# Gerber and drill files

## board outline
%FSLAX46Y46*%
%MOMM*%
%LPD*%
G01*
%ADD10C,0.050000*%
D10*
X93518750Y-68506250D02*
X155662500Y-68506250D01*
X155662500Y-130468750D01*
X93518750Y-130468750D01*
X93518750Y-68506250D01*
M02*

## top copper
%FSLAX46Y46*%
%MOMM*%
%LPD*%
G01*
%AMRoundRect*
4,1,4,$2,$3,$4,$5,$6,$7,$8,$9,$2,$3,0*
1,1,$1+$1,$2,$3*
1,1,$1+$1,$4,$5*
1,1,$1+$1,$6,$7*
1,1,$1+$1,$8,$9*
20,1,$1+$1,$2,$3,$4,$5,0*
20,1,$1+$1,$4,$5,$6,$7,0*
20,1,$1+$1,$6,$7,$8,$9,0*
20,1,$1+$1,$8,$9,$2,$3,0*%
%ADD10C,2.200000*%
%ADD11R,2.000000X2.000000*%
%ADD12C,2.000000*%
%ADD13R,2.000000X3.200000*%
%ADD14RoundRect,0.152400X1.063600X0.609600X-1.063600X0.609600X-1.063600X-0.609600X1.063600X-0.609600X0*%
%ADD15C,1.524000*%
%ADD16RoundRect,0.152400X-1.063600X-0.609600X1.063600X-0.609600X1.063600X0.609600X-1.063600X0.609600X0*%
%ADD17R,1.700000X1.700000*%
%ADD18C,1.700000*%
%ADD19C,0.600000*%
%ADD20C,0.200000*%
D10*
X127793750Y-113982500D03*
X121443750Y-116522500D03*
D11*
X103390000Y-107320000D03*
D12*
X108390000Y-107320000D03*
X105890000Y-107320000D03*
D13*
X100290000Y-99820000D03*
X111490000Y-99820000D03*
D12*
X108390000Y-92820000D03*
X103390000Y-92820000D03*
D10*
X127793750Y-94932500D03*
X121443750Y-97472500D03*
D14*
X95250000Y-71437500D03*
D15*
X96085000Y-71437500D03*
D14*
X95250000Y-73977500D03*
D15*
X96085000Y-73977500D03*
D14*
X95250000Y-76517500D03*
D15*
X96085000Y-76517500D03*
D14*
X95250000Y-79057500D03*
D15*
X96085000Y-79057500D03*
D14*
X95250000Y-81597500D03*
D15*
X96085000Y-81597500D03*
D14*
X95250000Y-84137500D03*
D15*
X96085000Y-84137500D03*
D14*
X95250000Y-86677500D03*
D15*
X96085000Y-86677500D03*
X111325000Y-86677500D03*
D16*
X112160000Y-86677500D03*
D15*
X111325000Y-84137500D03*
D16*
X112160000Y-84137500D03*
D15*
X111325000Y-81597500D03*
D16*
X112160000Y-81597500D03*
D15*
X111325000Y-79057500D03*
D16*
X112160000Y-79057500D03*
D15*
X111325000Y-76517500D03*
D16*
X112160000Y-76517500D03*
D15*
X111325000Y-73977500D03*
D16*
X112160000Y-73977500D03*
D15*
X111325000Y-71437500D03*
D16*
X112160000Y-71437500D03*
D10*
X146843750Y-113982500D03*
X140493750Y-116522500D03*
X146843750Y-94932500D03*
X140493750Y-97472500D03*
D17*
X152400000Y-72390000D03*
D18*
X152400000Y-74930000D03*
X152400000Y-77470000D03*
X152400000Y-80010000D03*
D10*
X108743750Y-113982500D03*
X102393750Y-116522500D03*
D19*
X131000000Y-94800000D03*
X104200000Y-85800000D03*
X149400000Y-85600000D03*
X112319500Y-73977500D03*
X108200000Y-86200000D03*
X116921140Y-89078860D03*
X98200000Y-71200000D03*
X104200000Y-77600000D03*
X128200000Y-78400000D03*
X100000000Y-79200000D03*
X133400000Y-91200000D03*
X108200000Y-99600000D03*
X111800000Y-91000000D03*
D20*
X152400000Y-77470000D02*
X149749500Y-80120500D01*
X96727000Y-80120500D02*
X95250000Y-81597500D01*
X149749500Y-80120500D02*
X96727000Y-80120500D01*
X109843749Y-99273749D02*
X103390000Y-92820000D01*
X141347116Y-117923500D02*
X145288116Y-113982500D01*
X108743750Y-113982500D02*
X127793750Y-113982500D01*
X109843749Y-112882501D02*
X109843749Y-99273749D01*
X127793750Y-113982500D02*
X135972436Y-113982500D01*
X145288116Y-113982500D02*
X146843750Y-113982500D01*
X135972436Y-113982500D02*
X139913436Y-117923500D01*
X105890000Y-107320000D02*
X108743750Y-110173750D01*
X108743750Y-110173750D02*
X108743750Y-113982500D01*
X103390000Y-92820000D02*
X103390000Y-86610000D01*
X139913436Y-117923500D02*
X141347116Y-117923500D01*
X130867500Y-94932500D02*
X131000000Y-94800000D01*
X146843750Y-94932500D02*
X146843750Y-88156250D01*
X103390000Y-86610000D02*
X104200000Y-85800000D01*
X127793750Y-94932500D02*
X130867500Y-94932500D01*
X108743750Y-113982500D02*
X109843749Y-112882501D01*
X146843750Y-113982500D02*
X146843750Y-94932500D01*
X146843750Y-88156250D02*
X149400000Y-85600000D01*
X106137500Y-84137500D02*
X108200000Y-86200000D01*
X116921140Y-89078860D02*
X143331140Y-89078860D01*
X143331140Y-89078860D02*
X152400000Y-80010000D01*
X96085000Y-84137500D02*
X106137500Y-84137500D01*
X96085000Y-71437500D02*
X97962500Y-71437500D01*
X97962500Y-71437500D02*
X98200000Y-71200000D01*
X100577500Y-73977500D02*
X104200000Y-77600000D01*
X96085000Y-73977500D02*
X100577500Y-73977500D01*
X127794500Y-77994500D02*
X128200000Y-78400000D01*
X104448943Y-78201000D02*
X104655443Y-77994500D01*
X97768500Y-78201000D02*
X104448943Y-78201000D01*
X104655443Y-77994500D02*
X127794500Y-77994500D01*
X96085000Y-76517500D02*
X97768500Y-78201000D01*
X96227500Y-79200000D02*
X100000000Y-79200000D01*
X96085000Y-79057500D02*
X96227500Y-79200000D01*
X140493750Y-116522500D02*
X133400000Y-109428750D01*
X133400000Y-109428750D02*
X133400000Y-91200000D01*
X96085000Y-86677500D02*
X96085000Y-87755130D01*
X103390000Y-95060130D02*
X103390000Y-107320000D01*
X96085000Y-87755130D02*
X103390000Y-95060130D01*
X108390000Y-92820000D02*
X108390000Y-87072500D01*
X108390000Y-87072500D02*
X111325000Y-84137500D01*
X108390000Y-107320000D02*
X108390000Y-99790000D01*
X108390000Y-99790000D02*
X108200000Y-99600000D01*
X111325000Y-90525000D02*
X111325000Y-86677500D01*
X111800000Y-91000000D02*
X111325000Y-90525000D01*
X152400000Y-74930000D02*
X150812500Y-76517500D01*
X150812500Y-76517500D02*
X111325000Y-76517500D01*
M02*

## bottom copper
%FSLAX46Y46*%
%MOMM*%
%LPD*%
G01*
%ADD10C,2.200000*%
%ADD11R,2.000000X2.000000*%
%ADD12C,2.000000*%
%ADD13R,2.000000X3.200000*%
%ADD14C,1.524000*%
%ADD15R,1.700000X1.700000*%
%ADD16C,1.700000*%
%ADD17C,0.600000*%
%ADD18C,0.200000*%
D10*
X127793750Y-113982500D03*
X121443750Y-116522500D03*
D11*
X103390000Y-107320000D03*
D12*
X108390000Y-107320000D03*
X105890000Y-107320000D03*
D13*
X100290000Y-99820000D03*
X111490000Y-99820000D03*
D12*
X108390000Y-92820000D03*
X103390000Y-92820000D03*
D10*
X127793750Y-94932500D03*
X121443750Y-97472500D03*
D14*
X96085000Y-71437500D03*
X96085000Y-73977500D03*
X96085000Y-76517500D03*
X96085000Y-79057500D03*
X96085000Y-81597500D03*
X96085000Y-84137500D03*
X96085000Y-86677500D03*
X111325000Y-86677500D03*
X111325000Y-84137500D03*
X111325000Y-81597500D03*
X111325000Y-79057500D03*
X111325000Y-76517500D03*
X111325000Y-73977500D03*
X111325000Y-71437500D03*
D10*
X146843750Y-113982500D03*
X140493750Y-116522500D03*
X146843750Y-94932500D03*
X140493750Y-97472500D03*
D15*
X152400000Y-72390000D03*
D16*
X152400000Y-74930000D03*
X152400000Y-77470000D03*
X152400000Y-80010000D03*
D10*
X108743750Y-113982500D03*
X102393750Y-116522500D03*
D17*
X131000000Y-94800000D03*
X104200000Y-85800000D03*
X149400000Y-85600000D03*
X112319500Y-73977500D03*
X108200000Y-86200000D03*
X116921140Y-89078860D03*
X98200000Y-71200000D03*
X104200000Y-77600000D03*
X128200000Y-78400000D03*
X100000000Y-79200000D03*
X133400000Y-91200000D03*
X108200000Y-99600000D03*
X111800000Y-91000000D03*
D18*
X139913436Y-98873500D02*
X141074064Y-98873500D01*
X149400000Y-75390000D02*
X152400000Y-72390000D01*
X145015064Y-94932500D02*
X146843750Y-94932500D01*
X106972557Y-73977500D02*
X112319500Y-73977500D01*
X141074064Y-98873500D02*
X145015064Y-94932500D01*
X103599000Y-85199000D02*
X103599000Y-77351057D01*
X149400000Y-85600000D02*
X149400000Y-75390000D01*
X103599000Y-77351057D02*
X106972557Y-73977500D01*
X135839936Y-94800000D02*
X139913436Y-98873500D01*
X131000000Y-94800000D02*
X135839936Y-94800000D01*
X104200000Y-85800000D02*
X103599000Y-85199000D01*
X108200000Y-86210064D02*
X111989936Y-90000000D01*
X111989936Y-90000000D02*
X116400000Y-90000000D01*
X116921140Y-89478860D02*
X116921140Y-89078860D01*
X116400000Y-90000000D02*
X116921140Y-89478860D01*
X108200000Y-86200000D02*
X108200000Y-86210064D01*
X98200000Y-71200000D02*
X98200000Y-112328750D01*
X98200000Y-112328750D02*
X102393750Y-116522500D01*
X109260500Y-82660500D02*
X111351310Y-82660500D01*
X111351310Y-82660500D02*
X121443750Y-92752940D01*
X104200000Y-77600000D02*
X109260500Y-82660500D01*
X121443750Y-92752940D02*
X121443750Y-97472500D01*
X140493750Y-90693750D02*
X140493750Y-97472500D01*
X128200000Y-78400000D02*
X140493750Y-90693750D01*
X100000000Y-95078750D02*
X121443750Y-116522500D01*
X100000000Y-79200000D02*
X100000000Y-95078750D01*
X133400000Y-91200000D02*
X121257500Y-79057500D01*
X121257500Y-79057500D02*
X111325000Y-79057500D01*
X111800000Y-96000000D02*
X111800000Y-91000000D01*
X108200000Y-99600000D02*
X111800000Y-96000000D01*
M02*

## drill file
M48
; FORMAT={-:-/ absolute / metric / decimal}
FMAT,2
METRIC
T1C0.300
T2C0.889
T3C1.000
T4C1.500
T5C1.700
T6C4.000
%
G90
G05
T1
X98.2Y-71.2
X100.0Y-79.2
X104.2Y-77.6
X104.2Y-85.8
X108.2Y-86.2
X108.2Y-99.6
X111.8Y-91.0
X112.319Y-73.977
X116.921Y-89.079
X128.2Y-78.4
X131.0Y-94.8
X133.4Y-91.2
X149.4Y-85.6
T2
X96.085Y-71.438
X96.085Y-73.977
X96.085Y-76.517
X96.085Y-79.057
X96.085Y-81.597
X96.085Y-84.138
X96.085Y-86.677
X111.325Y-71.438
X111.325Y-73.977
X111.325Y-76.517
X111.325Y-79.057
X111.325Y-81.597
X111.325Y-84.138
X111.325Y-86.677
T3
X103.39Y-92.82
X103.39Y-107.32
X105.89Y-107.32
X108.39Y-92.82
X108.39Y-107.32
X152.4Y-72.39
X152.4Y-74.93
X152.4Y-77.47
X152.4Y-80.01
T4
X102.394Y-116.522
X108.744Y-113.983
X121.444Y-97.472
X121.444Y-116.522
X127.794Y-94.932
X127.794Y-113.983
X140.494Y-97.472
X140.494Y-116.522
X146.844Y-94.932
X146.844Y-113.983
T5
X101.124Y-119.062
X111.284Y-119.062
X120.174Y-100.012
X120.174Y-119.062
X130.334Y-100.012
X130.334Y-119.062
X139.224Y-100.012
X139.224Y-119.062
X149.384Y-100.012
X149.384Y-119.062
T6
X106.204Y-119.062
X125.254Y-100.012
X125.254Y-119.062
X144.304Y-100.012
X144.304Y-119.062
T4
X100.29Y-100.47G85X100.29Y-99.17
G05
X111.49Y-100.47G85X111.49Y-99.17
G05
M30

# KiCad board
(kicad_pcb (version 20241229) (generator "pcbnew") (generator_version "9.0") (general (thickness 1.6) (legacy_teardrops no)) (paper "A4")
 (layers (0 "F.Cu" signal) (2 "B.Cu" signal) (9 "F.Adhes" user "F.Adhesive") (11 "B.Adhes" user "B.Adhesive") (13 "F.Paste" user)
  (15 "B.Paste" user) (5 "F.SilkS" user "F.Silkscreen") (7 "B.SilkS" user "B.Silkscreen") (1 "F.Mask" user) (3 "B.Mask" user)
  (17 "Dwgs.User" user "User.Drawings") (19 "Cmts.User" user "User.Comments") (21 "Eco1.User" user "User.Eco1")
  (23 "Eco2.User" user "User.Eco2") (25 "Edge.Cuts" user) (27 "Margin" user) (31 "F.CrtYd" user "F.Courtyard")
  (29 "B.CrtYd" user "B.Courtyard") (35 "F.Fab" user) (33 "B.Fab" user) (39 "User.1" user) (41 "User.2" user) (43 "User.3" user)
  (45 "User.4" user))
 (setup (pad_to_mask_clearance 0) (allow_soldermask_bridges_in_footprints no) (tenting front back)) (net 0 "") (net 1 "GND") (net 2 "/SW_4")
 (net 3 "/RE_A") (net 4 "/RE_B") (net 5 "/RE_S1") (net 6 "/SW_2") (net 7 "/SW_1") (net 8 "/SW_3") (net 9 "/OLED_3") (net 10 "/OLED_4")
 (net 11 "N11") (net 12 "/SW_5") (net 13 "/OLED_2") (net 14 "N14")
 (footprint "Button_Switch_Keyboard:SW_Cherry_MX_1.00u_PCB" (layer "F.Cu") (at 127.79375 113.9825)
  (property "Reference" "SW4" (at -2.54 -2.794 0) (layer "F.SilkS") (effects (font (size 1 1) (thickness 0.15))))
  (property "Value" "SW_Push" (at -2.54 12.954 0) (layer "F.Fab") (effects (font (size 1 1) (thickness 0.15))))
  (pad "" np_thru_hole circle (at -7.62 5.08) (size 1.7 1.7) (drill 1.7) (layers "*.Cu" "*.Mask"))
  (pad "" np_thru_hole circle (at -2.54 5.08) (size 4 4) (drill 4) (layers "*.Cu" "*.Mask"))
  (pad "" np_thru_hole circle (at 2.54 5.08) (size 1.7 1.7) (drill 1.7) (layers "*.Cu" "*.Mask"))
  (pad "1" thru_hole circle (at 0 0) (size 2.2 2.2) (drill 1.5) (layers "*.Cu" "*.Mask") (remove_unused_layers no) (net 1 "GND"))
  (pad "2" thru_hole circle (at -6.35 2.54) (size 2.2 2.2) (drill 1.5) (layers "*.Cu" "*.Mask") (remove_unused_layers no) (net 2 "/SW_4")))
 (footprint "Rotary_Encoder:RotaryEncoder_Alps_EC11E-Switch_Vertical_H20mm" (layer "F.Cu") (at 103.39 107.32 90)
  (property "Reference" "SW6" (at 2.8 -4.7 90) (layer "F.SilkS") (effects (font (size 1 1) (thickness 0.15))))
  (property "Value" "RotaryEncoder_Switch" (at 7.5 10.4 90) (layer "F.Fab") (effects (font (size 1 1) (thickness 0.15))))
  (pad "A" thru_hole rect (at 0 0 90) (size 2 2) (drill 1) (layers "*.Cu" "*.Mask") (remove_unused_layers no) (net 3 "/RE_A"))
  (pad "B" thru_hole circle (at 0 5 90) (size 2 2) (drill 1) (layers "*.Cu" "*.Mask") (remove_unused_layers no) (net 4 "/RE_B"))
  (pad "C" thru_hole circle (at 0 2.5 90) (size 2 2) (drill 1) (layers "*.Cu" "*.Mask") (remove_unused_layers no) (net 1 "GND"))
  (pad "MP" thru_hole rect (at 7.5 -3.1 90) (size 3.2 2) (drill oval 2.8 1.5) (layers "*.Cu" "*.Mask") (remove_unused_layers no))
  (pad "MP" thru_hole rect (at 7.5 8.1 90) (size 3.2 2) (drill oval 2.8 1.5) (layers "*.Cu" "*.Mask") (remove_unused_layers no))
  (pad "S1" thru_hole circle (at 14.5 5 90) (size 2 2) (drill 1) (layers "*.Cu" "*.Mask") (remove_unused_layers no) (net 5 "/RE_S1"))
  (pad "S2" thru_hole circle (at 14.5 0 90) (size 2 2) (drill 1) (layers "*.Cu" "*.Mask") (remove_unused_layers no) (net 1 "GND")))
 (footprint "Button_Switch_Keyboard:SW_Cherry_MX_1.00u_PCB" (layer "F.Cu") (at 127.79375 94.9325)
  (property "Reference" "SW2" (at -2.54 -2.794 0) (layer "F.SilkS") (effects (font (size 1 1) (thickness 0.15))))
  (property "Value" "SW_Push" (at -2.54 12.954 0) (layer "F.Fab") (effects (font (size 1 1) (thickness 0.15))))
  (pad "" np_thru_hole circle (at -7.62 5.08) (size 1.7 1.7) (drill 1.7) (layers "*.Cu" "*.Mask"))
  (pad "" np_thru_hole circle (at -2.54 5.08) (size 4 4) (drill 4) (layers "*.Cu" "*.Mask"))
  (pad "" np_thru_hole circle (at 2.54 5.08) (size 1.7 1.7) (drill 1.7) (layers "*.Cu" "*.Mask"))
  (pad "1" thru_hole circle (at 0 0) (size 2.2 2.2) (drill 1.5) (layers "*.Cu" "*.Mask") (remove_unused_layers no) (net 1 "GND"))
  (pad "2" thru_hole circle (at -6.35 2.54) (size 2.2 2.2) (drill 1.5) (layers "*.Cu" "*.Mask") (remove_unused_layers no) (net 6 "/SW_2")))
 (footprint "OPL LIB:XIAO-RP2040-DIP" (layer "F.Cu") (at 103.705 79.0575)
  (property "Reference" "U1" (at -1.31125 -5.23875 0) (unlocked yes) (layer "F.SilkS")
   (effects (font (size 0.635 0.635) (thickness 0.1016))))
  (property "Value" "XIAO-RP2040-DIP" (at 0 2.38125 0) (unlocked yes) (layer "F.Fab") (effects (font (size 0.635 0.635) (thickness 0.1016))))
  (pad "1" smd roundrect (at -8.455 -7.62 180) (size 2.432 1.524) (layers "F.Cu" "F.Mask") (roundrect_rratio 0.1) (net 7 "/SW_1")
   (thermal_bridge_angle 45))
  (pad "1" thru_hole circle (at -7.62 -7.62 180) (size 1.524 1.524) (drill 0.889) (layers "*.Cu" "*.Mask") (remove_unused_layers no)
   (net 7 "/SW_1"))
  (pad "2" smd roundrect (at -8.455 -5.08 180) (size 2.432 1.524) (layers "F.Cu" "F.Mask") (roundrect_rratio 0.1) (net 6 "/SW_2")
   (thermal_bridge_angle 45))
  (pad "2" thru_hole circle (at -7.62 -5.08 180) (size 1.524 1.524) (drill 0.889) (layers "*.Cu" "*.Mask") (remove_unused_layers no)
   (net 6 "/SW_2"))
  (pad "3" smd roundrect (at -8.455 -2.54 180) (size 2.432 1.524) (layers "F.Cu" "F.Mask") (roundrect_rratio 0.1) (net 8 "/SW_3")
   (thermal_bridge_angle 45))
  (pad "3" thru_hole circle (at -7.62 -2.54 180) (size 1.524 1.524) (drill 0.889) (layers "*.Cu" "*.Mask") (remove_unused_layers no)
   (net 8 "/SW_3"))
  (pad "4" smd roundrect (at -8.455 0 180) (size 2.432 1.524) (layers "F.Cu" "F.Mask") (roundrect_rratio 0.1) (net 2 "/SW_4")
   (thermal_bridge_angle 45))
  (pad "4" thru_hole circle (at -7.62 0 180) (size 1.524 1.524) (drill 0.889) (layers "*.Cu" "*.Mask") (remove_unused_layers no)
   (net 2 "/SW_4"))
  (pad "5" smd roundrect (at -8.455 2.54 180) (size 2.432 1.524) (layers "F.Cu" "F.Mask") (roundrect_rratio 0.1) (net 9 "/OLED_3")
   (thermal_bridge_angle 45))
  (pad "5" thru_hole circle (at -7.62 2.54 180) (size 1.524 1.524) (drill 0.889) (layers "*.Cu" "*.Mask") (remove_unused_layers no)
   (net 9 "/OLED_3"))
  (pad "6" smd roundrect (at -8.455 5.08 180) (size 2.432 1.524) (layers "F.Cu" "F.Mask") (roundrect_rratio 0.1) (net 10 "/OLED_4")
   (thermal_bridge_angle 45))
  (pad "6" thru_hole circle (at -7.62 5.08 180) (size 1.524 1.524) (drill 0.889) (layers "*.Cu" "*.Mask") (remove_unused_layers no)
   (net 10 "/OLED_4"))
  (pad "7" smd roundrect (at -8.455 7.62 180) (size 2.432 1.524) (layers "F.Cu" "F.Mask") (roundrect_rratio 0.1) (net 3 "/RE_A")
   (thermal_bridge_angle 45))
  (pad "7" thru_hole circle (at -7.62 7.62 180) (size 1.524 1.524) (drill 0.889) (layers "*.Cu" "*.Mask") (remove_unused_layers no)
   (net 3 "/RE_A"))
  (pad "8" thru_hole circle (at 7.62 7.62) (size 1.524 1.524) (drill 0.889) (layers "*.Cu" "*.Mask") (remove_unused_layers no)
   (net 4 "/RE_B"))
  (pad "8" smd roundrect (at 8.455 7.62) (size 2.432 1.524) (layers "F.Cu" "F.Mask") (roundrect_rratio 0.1) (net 4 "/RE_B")
   (thermal_bridge_angle 45))
  (pad "9" thru_hole circle (at 7.62 5.08) (size 1.524 1.524) (drill 0.889) (layers "*.Cu" "*.Mask") (remove_unused_layers no)
   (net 5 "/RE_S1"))
  (pad "9" smd roundrect (at 8.455 5.08) (size 2.432 1.524) (layers "F.Cu" "F.Mask") (roundrect_rratio 0.1) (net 5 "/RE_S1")
   (thermal_bridge_angle 45))
  (pad "10" thru_hole circle (at 7.62 2.54) (size 1.524 1.524) (drill 0.889) (layers "*.Cu" "*.Mask") (remove_unused_layers no)
   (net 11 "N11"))
  (pad "10" smd roundrect (at 8.455 2.54) (size 2.432 1.524) (layers "F.Cu" "F.Mask") (roundrect_rratio 0.1) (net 11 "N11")
   (thermal_bridge_angle 45))
  (pad "11" thru_hole circle (at 7.62 0) (size 1.524 1.524) (drill 0.889) (layers "*.Cu" "*.Mask") (remove_unused_layers no)
   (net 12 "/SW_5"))
  (pad "11" smd roundrect (at 8.455 0) (size 2.432 1.524) (layers "F.Cu" "F.Mask") (roundrect_rratio 0.1) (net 12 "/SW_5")
   (thermal_bridge_angle 45))
  (pad "12" thru_hole circle (at 7.62 -2.54) (size 1.524 1.524) (drill 0.889) (layers "*.Cu" "*.Mask") (remove_unused_layers no)
   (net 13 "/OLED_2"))
  (pad "12" smd roundrect (at 8.455 -2.54) (size 2.432 1.524) (layers "F.Cu" "F.Mask") (roundrect_rratio 0.1) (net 13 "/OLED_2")
   (thermal_bridge_angle 45))
  (pad "13" thru_hole circle (at 7.62 -5.08) (size 1.524 1.524) (drill 0.889) (layers "*.Cu" "*.Mask") (remove_unused_layers no)
   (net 1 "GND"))
  (pad "13" smd roundrect (at 8.455 -5.08) (size 2.432 1.524) (layers "F.Cu" "F.Mask") (roundrect_rratio 0.1) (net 1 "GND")
   (thermal_bridge_angle 45))
  (pad "14" thru_hole circle (at 7.62 -7.62) (size 1.524 1.524) (drill 0.889) (layers "*.Cu" "*.Mask") (remove_unused_layers no)
   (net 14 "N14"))
  (pad "14" smd roundrect (at 8.455 -7.62) (size 2.432 1.524) (layers "F.Cu" "F.Mask") (roundrect_rratio 0.1) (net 14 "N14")
   (thermal_bridge_angle 45)))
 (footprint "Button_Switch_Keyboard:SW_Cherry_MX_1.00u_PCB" (layer "F.Cu") (at 146.84375 113.9825)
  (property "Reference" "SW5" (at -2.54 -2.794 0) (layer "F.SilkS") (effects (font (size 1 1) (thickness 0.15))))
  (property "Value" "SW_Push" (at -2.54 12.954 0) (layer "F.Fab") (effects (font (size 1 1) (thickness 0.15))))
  (pad "" np_thru_hole circle (at -7.62 5.08) (size 1.7 1.7) (drill 1.7) (layers "*.Cu" "*.Mask"))
  (pad "" np_thru_hole circle (at -2.54 5.08) (size 4 4) (drill 4) (layers "*.Cu" "*.Mask"))
  (pad "" np_thru_hole circle (at 2.54 5.08) (size 1.7 1.7) (drill 1.7) (layers "*.Cu" "*.Mask"))
  (pad "1" thru_hole circle (at 0 0) (size 2.2 2.2) (drill 1.5) (layers "*.Cu" "*.Mask") (remove_unused_layers no) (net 1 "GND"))
  (pad "2" thru_hole circle (at -6.35 2.54) (size 2.2 2.2) (drill 1.5) (layers "*.Cu" "*.Mask") (remove_unused_layers no) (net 12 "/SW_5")))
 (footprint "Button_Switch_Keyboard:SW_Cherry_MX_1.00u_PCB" (layer "F.Cu") (at 146.84375 94.9325)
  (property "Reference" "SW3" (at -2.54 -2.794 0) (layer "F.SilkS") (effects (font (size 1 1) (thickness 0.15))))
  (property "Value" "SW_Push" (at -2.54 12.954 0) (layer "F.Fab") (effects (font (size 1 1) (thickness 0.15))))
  (pad "" np_thru_hole circle (at -7.62 5.08) (size 1.7 1.7) (drill 1.7) (layers "*.Cu" "*.Mask"))
  (pad "" np_thru_hole circle (at -2.54 5.08) (size 4 4) (drill 4) (layers "*.Cu" "*.Mask"))
  (pad "" np_thru_hole circle (at 2.54 5.08) (size 1.7 1.7) (drill 1.7) (layers "*.Cu" "*.Mask"))
  (pad "1" thru_hole circle (at 0 0) (size 2.2 2.2) (drill 1.5) (layers "*.Cu" "*.Mask") (remove_unused_layers no) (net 1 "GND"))
  (pad "2" thru_hole circle (at -6.35 2.54) (size 2.2 2.2) (drill 1.5) (layers "*.Cu" "*.Mask") (remove_unused_layers no) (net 8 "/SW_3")))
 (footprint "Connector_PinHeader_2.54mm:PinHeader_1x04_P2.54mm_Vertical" (layer "F.Cu") (at 152.4 72.39)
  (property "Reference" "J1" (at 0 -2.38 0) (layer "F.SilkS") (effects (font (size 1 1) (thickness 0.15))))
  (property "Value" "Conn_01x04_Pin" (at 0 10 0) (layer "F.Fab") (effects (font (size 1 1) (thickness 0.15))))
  (pad "1" thru_hole rect (at 0 0) (size 1.7 1.7) (drill 1) (layers "*.Cu" "*.Mask") (remove_unused_layers no) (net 1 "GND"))
  (pad "2" thru_hole circle (at 0 2.54) (size 1.7 1.7) (drill 1) (layers "*.Cu" "*.Mask") (remove_unused_layers no) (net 13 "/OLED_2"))
  (pad "3" thru_hole circle (at 0 5.08) (size 1.7 1.7) (drill 1) (layers "*.Cu" "*.Mask") (remove_unused_layers no) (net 9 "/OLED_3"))
  (pad "4" thru_hole circle (at 0 7.62) (size 1.7 1.7) (drill 1) (layers "*.Cu" "*.Mask") (remove_unused_layers no) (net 10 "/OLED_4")))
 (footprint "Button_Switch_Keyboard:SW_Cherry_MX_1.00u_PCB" (layer "F.Cu") (at 108.74375 113.9825)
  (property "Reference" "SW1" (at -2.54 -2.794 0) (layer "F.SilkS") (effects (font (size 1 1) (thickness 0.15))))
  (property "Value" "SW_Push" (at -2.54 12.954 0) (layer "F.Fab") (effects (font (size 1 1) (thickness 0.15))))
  (pad "" np_thru_hole circle (at -7.62 5.08) (size 1.7 1.7) (drill 1.7) (layers "*.Cu" "*.Mask"))
  (pad "" np_thru_hole circle (at -2.54 5.08) (size 4 4) (drill 4) (layers "*.Cu" "*.Mask"))
  (pad "" np_thru_hole circle (at 2.54 5.08) (size 1.7 1.7) (drill 1.7) (layers "*.Cu" "*.Mask"))
  (pad "1" thru_hole circle (at 0 0) (size 2.2 2.2) (drill 1.5) (layers "*.Cu" "*.Mask") (remove_unused_layers no) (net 1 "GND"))
  (pad "2" thru_hole circle (at -6.35 2.54) (size 2.2 2.2) (drill 1.5) (layers "*.Cu" "*.Mask") (remove_unused_layers no) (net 7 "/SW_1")))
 (gr_rect (start 93.51875 68.50625) (end 155.6625 130.46875) (stroke (width 0.05) (type default)) (fill no) (layer "Edge.Cuts"))
 (segment (start 152.4 77.47) (end 149.7495 80.1205) (width 0.2) (layer "F.Cu") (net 9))
 (segment (start 96.727 80.1205) (end 95.25 81.5975) (width 0.2) (layer "F.Cu") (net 9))
 (segment (start 149.7495 80.1205) (end 96.727 80.1205) (width 0.2) (layer "F.Cu") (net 9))
 (segment (start 109.843749 99.273749) (end 103.39 92.82) (width 0.2) (layer "F.Cu") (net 1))
 (segment (start 141.347116 117.9235) (end 145.288116 113.9825) (width 0.2) (layer "F.Cu") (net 1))
 (segment (start 108.74375 113.9825) (end 127.79375 113.9825) (width 0.2) (layer "F.Cu") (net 1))
 (segment (start 109.843749 112.882501) (end 109.843749 99.273749) (width 0.2) (layer "F.Cu") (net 1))
 (segment (start 127.79375 113.9825) (end 135.972436 113.9825) (width 0.2) (layer "F.Cu") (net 1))
 (segment (start 145.288116 113.9825) (end 146.84375 113.9825) (width 0.2) (layer "F.Cu") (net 1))
 (segment (start 135.972436 113.9825) (end 139.913436 117.9235) (width 0.2) (layer "F.Cu") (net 1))
 (segment (start 105.89 107.32) (end 108.74375 110.17375) (width 0.2) (layer "F.Cu") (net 1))
 (segment (start 108.74375 110.17375) (end 108.74375 113.9825) (width 0.2) (layer "F.Cu") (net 1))
 (segment (start 103.39 92.82) (end 103.39 86.61) (width 0.2) (layer "F.Cu") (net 1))
 (segment (start 139.913436 117.9235) (end 141.347116 117.9235) (width 0.2) (layer "F.Cu") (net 1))
 (segment (start 130.8675 94.9325) (end 131 94.8) (width 0.2) (layer "F.Cu") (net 1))
 (segment (start 146.84375 94.9325) (end 146.84375 88.15625) (width 0.2) (layer "F.Cu") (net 1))
 (segment (start 103.39 86.61) (end 104.2 85.8) (width 0.2) (layer "F.Cu") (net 1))
 (segment (start 127.79375 94.9325) (end 130.8675 94.9325) (width 0.2) (layer "F.Cu") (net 1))
 (segment (start 108.74375 113.9825) (end 109.843749 112.882501) (width 0.2) (layer "F.Cu") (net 1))
 (segment (start 146.84375 113.9825) (end 146.84375 94.9325) (width 0.2) (layer "F.Cu") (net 1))
 (segment (start 146.84375 88.15625) (end 149.4 85.6) (width 0.2) (layer "F.Cu") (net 1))
 (via (at 131 94.8) (size 0.6) (drill 0.3) (layers "F.Cu" "B.Cu") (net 1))
 (via (at 104.2 85.8) (size 0.6) (drill 0.3) (layers "F.Cu" "B.Cu") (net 1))
 (via (at 149.4 85.6) (size 0.6) (drill 0.3) (layers "F.Cu" "B.Cu") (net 1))
 (via (at 112.3195 73.9775) (size 0.6) (drill 0.3) (layers "F.Cu" "B.Cu") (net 1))
 (segment (start 139.913436 98.8735) (end 141.074064 98.8735) (width 0.2) (layer "B.Cu") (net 1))
 (segment (start 149.4 75.39) (end 152.4 72.39) (width 0.2) (layer "B.Cu") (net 1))
 (segment (start 145.015064 94.9325) (end 146.84375 94.9325) (width 0.2) (layer "B.Cu") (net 1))
 (segment (start 106.972557 73.9775) (end 112.3195 73.9775) (width 0.2) (layer "B.Cu") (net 1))
 (segment (start 141.074064 98.8735) (end 145.015064 94.9325) (width 0.2) (layer "B.Cu") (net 1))
 (segment (start 103.599 85.199) (end 103.599 77.351057) (width 0.2) (layer "B.Cu") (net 1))
 (segment (start 149.4 85.6) (end 149.4 75.39) (width 0.2) (layer "B.Cu") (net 1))
 (segment (start 103.599 77.351057) (end 106.972557 73.9775) (width 0.2) (layer "B.Cu") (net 1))
 (segment (start 135.839936 94.8) (end 139.913436 98.8735) (width 0.2) (layer "B.Cu") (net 1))
 (segment (start 131 94.8) (end 135.839936 94.8) (width 0.2) (layer "B.Cu") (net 1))
 (segment (start 104.2 85.8) (end 103.599 85.199) (width 0.2) (layer "B.Cu") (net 1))
 (segment (start 106.1375 84.1375) (end 108.2 86.2) (width 0.2) (layer "F.Cu") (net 10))
 (segment (start 116.92114 89.07886) (end 143.33114 89.07886) (width 0.2) (layer "F.Cu") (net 10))
 (segment (start 143.33114 89.07886) (end 152.4 80.01) (width 0.2) (layer "F.Cu") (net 10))
 (segment (start 96.085 84.1375) (end 106.1375 84.1375) (width 0.2) (layer "F.Cu") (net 10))
 (via (at 108.2 86.2) (size 0.6) (drill 0.3) (layers "F.Cu" "B.Cu") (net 10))
 (via (at 116.92114 89.07886) (size 0.6) (drill 0.3) (layers "F.Cu" "B.Cu") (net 10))
 (segment (start 108.2 86.210064) (end 111.989936 90) (width 0.2) (layer "B.Cu") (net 10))
 (segment (start 111.989936 90) (end 116.4 90) (width 0.2) (layer "B.Cu") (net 10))
 (segment (start 116.92114 89.47886) (end 116.92114 89.07886) (width 0.2) (layer "B.Cu") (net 10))
 (segment (start 116.4 90) (end 116.92114 89.47886) (width 0.2) (layer "B.Cu") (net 10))
 (segment (start 108.2 86.2) (end 108.2 86.210064) (width 0.2) (layer "B.Cu") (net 10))
 (segment (start 96.085 71.4375) (end 97.9625 71.4375) (width 0.2) (layer "F.Cu") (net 7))
 (segment (start 97.9625 71.4375) (end 98.2 71.2) (width 0.2) (layer "F.Cu") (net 7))
 (via (at 98.2 71.2) (size 0.6) (drill 0.3) (layers "F.Cu" "B.Cu") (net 7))
 (segment (start 98.2 71.2) (end 98.2 112.32875) (width 0.2) (layer "B.Cu") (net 7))
 (segment (start 98.2 112.32875) (end 102.39375 116.5225) (width 0.2) (layer "B.Cu") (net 7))
 (segment (start 100.5775 73.9775) (end 104.2 77.6) (width 0.2) (layer "F.Cu") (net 6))
 (segment (start 96.085 73.9775) (end 100.5775 73.9775) (width 0.2) (layer "F.Cu") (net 6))
 (via (at 104.2 77.6) (size 0.6) (drill 0.3) (layers "F.Cu" "B.Cu") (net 6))
 (segment (start 109.2605 82.6605) (end 111.35131 82.6605) (width 0.2) (layer "B.Cu") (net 6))
 (segment (start 111.35131 82.6605) (end 121.44375 92.75294) (width 0.2) (layer "B.Cu") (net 6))
 (segment (start 104.2 77.6) (end 109.2605 82.6605) (width 0.2) (layer "B.Cu") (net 6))
 (segment (start 121.44375 92.75294) (end 121.44375 97.4725) (width 0.2) (layer "B.Cu") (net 6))
 (segment (start 127.7945 77.9945) (end 128.2 78.4) (width 0.2) (layer "F.Cu") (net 8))
 (segment (start 104.448943 78.201) (end 104.655443 77.9945) (width 0.2) (layer "F.Cu") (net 8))
 (segment (start 97.7685 78.201) (end 104.448943 78.201) (width 0.2) (layer "F.Cu") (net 8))
 (segment (start 104.655443 77.9945) (end 127.7945 77.9945) (width 0.2) (layer "F.Cu") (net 8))
 (segment (start 96.085 76.5175) (end 97.7685 78.201) (width 0.2) (layer "F.Cu") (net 8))
 (via (at 128.2 78.4) (size 0.6) (drill 0.3) (layers "F.Cu" "B.Cu") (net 8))
 (segment (start 140.49375 90.69375) (end 140.49375 97.4725) (width 0.2) (layer "B.Cu") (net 8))
 (segment (start 128.2 78.4) (end 140.49375 90.69375) (width 0.2) (layer "B.Cu") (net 8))
 (segment (start 96.2275 79.2) (end 100 79.2) (width 0.2) (layer "F.Cu") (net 2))
 (segment (start 96.085 79.0575) (end 96.2275 79.2) (width 0.2) (layer "F.Cu") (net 2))
 (via (at 100 79.2) (size 0.6) (drill 0.3) (layers "F.Cu" "B.Cu") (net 2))
 (segment (start 100 95.07875) (end 121.44375 116.5225) (width 0.2) (layer "B.Cu") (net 2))
 (segment (start 100 79.2) (end 100 95.07875) (width 0.2) (layer "B.Cu") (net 2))
 (segment (start 140.49375 116.5225) (end 133.4 109.42875) (width 0.2) (layer "F.Cu") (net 12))
 (segment (start 133.4 109.42875) (end 133.4 91.2) (width 0.2) (layer "F.Cu") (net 12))
 (via (at 133.4 91.2) (size 0.6) (drill 0.3) (layers "F.Cu" "B.Cu") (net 12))
 (segment (start 133.4 91.2) (end 121.2575 79.0575) (width 0.2) (layer "B.Cu") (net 12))
 (segment (start 121.2575 79.0575) (end 111.325 79.0575) (width 0.2) (layer "B.Cu") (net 12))
 (segment (start 96.085 86.6775) (end 96.085 87.75513) (width 0.2) (layer "F.Cu") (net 3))
 (segment (start 103.39 95.06013) (end 103.39 107.32) (width 0.2) (layer "F.Cu") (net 3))
 (segment (start 96.085 87.75513) (end 103.39 95.06013) (width 0.2) (layer "F.Cu") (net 3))
 (segment (start 108.39 92.82) (end 108.39 87.0725) (width 0.2) (layer "F.Cu") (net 5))
 (segment (start 108.39 87.0725) (end 111.325 84.1375) (width 0.2) (layer "F.Cu") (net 5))
 (segment (start 108.39 107.32) (end 108.39 99.79) (width 0.2) (layer "F.Cu") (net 4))
 (segment (start 108.39 99.79) (end 108.2 99.6) (width 0.2) (layer "F.Cu") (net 4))
 (segment (start 111.325 90.525) (end 111.325 86.6775) (width 0.2) (layer "F.Cu") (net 4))
 (segment (start 111.8 91) (end 111.325 90.525) (width 0.2) (layer "F.Cu") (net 4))
 (via (at 108.2 99.6) (size 0.6) (drill 0.3) (layers "F.Cu" "B.Cu") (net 4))
 (via (at 111.8 91) (size 0.6) (drill 0.3) (layers "F.Cu" "B.Cu") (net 4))
 (segment (start 111.8 96) (end 111.8 91) (width 0.2) (layer "B.Cu") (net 4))
 (segment (start 108.2 99.6) (end 111.8 96) (width 0.2) (layer "B.Cu") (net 4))
 (segment (start 152.4 74.93) (end 150.8125 76.5175) (width 0.2) (layer "F.Cu") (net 13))
 (segment (start 150.8125 76.5175) (end 111.325 76.5175) (width 0.2) (layer "F.Cu") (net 13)))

